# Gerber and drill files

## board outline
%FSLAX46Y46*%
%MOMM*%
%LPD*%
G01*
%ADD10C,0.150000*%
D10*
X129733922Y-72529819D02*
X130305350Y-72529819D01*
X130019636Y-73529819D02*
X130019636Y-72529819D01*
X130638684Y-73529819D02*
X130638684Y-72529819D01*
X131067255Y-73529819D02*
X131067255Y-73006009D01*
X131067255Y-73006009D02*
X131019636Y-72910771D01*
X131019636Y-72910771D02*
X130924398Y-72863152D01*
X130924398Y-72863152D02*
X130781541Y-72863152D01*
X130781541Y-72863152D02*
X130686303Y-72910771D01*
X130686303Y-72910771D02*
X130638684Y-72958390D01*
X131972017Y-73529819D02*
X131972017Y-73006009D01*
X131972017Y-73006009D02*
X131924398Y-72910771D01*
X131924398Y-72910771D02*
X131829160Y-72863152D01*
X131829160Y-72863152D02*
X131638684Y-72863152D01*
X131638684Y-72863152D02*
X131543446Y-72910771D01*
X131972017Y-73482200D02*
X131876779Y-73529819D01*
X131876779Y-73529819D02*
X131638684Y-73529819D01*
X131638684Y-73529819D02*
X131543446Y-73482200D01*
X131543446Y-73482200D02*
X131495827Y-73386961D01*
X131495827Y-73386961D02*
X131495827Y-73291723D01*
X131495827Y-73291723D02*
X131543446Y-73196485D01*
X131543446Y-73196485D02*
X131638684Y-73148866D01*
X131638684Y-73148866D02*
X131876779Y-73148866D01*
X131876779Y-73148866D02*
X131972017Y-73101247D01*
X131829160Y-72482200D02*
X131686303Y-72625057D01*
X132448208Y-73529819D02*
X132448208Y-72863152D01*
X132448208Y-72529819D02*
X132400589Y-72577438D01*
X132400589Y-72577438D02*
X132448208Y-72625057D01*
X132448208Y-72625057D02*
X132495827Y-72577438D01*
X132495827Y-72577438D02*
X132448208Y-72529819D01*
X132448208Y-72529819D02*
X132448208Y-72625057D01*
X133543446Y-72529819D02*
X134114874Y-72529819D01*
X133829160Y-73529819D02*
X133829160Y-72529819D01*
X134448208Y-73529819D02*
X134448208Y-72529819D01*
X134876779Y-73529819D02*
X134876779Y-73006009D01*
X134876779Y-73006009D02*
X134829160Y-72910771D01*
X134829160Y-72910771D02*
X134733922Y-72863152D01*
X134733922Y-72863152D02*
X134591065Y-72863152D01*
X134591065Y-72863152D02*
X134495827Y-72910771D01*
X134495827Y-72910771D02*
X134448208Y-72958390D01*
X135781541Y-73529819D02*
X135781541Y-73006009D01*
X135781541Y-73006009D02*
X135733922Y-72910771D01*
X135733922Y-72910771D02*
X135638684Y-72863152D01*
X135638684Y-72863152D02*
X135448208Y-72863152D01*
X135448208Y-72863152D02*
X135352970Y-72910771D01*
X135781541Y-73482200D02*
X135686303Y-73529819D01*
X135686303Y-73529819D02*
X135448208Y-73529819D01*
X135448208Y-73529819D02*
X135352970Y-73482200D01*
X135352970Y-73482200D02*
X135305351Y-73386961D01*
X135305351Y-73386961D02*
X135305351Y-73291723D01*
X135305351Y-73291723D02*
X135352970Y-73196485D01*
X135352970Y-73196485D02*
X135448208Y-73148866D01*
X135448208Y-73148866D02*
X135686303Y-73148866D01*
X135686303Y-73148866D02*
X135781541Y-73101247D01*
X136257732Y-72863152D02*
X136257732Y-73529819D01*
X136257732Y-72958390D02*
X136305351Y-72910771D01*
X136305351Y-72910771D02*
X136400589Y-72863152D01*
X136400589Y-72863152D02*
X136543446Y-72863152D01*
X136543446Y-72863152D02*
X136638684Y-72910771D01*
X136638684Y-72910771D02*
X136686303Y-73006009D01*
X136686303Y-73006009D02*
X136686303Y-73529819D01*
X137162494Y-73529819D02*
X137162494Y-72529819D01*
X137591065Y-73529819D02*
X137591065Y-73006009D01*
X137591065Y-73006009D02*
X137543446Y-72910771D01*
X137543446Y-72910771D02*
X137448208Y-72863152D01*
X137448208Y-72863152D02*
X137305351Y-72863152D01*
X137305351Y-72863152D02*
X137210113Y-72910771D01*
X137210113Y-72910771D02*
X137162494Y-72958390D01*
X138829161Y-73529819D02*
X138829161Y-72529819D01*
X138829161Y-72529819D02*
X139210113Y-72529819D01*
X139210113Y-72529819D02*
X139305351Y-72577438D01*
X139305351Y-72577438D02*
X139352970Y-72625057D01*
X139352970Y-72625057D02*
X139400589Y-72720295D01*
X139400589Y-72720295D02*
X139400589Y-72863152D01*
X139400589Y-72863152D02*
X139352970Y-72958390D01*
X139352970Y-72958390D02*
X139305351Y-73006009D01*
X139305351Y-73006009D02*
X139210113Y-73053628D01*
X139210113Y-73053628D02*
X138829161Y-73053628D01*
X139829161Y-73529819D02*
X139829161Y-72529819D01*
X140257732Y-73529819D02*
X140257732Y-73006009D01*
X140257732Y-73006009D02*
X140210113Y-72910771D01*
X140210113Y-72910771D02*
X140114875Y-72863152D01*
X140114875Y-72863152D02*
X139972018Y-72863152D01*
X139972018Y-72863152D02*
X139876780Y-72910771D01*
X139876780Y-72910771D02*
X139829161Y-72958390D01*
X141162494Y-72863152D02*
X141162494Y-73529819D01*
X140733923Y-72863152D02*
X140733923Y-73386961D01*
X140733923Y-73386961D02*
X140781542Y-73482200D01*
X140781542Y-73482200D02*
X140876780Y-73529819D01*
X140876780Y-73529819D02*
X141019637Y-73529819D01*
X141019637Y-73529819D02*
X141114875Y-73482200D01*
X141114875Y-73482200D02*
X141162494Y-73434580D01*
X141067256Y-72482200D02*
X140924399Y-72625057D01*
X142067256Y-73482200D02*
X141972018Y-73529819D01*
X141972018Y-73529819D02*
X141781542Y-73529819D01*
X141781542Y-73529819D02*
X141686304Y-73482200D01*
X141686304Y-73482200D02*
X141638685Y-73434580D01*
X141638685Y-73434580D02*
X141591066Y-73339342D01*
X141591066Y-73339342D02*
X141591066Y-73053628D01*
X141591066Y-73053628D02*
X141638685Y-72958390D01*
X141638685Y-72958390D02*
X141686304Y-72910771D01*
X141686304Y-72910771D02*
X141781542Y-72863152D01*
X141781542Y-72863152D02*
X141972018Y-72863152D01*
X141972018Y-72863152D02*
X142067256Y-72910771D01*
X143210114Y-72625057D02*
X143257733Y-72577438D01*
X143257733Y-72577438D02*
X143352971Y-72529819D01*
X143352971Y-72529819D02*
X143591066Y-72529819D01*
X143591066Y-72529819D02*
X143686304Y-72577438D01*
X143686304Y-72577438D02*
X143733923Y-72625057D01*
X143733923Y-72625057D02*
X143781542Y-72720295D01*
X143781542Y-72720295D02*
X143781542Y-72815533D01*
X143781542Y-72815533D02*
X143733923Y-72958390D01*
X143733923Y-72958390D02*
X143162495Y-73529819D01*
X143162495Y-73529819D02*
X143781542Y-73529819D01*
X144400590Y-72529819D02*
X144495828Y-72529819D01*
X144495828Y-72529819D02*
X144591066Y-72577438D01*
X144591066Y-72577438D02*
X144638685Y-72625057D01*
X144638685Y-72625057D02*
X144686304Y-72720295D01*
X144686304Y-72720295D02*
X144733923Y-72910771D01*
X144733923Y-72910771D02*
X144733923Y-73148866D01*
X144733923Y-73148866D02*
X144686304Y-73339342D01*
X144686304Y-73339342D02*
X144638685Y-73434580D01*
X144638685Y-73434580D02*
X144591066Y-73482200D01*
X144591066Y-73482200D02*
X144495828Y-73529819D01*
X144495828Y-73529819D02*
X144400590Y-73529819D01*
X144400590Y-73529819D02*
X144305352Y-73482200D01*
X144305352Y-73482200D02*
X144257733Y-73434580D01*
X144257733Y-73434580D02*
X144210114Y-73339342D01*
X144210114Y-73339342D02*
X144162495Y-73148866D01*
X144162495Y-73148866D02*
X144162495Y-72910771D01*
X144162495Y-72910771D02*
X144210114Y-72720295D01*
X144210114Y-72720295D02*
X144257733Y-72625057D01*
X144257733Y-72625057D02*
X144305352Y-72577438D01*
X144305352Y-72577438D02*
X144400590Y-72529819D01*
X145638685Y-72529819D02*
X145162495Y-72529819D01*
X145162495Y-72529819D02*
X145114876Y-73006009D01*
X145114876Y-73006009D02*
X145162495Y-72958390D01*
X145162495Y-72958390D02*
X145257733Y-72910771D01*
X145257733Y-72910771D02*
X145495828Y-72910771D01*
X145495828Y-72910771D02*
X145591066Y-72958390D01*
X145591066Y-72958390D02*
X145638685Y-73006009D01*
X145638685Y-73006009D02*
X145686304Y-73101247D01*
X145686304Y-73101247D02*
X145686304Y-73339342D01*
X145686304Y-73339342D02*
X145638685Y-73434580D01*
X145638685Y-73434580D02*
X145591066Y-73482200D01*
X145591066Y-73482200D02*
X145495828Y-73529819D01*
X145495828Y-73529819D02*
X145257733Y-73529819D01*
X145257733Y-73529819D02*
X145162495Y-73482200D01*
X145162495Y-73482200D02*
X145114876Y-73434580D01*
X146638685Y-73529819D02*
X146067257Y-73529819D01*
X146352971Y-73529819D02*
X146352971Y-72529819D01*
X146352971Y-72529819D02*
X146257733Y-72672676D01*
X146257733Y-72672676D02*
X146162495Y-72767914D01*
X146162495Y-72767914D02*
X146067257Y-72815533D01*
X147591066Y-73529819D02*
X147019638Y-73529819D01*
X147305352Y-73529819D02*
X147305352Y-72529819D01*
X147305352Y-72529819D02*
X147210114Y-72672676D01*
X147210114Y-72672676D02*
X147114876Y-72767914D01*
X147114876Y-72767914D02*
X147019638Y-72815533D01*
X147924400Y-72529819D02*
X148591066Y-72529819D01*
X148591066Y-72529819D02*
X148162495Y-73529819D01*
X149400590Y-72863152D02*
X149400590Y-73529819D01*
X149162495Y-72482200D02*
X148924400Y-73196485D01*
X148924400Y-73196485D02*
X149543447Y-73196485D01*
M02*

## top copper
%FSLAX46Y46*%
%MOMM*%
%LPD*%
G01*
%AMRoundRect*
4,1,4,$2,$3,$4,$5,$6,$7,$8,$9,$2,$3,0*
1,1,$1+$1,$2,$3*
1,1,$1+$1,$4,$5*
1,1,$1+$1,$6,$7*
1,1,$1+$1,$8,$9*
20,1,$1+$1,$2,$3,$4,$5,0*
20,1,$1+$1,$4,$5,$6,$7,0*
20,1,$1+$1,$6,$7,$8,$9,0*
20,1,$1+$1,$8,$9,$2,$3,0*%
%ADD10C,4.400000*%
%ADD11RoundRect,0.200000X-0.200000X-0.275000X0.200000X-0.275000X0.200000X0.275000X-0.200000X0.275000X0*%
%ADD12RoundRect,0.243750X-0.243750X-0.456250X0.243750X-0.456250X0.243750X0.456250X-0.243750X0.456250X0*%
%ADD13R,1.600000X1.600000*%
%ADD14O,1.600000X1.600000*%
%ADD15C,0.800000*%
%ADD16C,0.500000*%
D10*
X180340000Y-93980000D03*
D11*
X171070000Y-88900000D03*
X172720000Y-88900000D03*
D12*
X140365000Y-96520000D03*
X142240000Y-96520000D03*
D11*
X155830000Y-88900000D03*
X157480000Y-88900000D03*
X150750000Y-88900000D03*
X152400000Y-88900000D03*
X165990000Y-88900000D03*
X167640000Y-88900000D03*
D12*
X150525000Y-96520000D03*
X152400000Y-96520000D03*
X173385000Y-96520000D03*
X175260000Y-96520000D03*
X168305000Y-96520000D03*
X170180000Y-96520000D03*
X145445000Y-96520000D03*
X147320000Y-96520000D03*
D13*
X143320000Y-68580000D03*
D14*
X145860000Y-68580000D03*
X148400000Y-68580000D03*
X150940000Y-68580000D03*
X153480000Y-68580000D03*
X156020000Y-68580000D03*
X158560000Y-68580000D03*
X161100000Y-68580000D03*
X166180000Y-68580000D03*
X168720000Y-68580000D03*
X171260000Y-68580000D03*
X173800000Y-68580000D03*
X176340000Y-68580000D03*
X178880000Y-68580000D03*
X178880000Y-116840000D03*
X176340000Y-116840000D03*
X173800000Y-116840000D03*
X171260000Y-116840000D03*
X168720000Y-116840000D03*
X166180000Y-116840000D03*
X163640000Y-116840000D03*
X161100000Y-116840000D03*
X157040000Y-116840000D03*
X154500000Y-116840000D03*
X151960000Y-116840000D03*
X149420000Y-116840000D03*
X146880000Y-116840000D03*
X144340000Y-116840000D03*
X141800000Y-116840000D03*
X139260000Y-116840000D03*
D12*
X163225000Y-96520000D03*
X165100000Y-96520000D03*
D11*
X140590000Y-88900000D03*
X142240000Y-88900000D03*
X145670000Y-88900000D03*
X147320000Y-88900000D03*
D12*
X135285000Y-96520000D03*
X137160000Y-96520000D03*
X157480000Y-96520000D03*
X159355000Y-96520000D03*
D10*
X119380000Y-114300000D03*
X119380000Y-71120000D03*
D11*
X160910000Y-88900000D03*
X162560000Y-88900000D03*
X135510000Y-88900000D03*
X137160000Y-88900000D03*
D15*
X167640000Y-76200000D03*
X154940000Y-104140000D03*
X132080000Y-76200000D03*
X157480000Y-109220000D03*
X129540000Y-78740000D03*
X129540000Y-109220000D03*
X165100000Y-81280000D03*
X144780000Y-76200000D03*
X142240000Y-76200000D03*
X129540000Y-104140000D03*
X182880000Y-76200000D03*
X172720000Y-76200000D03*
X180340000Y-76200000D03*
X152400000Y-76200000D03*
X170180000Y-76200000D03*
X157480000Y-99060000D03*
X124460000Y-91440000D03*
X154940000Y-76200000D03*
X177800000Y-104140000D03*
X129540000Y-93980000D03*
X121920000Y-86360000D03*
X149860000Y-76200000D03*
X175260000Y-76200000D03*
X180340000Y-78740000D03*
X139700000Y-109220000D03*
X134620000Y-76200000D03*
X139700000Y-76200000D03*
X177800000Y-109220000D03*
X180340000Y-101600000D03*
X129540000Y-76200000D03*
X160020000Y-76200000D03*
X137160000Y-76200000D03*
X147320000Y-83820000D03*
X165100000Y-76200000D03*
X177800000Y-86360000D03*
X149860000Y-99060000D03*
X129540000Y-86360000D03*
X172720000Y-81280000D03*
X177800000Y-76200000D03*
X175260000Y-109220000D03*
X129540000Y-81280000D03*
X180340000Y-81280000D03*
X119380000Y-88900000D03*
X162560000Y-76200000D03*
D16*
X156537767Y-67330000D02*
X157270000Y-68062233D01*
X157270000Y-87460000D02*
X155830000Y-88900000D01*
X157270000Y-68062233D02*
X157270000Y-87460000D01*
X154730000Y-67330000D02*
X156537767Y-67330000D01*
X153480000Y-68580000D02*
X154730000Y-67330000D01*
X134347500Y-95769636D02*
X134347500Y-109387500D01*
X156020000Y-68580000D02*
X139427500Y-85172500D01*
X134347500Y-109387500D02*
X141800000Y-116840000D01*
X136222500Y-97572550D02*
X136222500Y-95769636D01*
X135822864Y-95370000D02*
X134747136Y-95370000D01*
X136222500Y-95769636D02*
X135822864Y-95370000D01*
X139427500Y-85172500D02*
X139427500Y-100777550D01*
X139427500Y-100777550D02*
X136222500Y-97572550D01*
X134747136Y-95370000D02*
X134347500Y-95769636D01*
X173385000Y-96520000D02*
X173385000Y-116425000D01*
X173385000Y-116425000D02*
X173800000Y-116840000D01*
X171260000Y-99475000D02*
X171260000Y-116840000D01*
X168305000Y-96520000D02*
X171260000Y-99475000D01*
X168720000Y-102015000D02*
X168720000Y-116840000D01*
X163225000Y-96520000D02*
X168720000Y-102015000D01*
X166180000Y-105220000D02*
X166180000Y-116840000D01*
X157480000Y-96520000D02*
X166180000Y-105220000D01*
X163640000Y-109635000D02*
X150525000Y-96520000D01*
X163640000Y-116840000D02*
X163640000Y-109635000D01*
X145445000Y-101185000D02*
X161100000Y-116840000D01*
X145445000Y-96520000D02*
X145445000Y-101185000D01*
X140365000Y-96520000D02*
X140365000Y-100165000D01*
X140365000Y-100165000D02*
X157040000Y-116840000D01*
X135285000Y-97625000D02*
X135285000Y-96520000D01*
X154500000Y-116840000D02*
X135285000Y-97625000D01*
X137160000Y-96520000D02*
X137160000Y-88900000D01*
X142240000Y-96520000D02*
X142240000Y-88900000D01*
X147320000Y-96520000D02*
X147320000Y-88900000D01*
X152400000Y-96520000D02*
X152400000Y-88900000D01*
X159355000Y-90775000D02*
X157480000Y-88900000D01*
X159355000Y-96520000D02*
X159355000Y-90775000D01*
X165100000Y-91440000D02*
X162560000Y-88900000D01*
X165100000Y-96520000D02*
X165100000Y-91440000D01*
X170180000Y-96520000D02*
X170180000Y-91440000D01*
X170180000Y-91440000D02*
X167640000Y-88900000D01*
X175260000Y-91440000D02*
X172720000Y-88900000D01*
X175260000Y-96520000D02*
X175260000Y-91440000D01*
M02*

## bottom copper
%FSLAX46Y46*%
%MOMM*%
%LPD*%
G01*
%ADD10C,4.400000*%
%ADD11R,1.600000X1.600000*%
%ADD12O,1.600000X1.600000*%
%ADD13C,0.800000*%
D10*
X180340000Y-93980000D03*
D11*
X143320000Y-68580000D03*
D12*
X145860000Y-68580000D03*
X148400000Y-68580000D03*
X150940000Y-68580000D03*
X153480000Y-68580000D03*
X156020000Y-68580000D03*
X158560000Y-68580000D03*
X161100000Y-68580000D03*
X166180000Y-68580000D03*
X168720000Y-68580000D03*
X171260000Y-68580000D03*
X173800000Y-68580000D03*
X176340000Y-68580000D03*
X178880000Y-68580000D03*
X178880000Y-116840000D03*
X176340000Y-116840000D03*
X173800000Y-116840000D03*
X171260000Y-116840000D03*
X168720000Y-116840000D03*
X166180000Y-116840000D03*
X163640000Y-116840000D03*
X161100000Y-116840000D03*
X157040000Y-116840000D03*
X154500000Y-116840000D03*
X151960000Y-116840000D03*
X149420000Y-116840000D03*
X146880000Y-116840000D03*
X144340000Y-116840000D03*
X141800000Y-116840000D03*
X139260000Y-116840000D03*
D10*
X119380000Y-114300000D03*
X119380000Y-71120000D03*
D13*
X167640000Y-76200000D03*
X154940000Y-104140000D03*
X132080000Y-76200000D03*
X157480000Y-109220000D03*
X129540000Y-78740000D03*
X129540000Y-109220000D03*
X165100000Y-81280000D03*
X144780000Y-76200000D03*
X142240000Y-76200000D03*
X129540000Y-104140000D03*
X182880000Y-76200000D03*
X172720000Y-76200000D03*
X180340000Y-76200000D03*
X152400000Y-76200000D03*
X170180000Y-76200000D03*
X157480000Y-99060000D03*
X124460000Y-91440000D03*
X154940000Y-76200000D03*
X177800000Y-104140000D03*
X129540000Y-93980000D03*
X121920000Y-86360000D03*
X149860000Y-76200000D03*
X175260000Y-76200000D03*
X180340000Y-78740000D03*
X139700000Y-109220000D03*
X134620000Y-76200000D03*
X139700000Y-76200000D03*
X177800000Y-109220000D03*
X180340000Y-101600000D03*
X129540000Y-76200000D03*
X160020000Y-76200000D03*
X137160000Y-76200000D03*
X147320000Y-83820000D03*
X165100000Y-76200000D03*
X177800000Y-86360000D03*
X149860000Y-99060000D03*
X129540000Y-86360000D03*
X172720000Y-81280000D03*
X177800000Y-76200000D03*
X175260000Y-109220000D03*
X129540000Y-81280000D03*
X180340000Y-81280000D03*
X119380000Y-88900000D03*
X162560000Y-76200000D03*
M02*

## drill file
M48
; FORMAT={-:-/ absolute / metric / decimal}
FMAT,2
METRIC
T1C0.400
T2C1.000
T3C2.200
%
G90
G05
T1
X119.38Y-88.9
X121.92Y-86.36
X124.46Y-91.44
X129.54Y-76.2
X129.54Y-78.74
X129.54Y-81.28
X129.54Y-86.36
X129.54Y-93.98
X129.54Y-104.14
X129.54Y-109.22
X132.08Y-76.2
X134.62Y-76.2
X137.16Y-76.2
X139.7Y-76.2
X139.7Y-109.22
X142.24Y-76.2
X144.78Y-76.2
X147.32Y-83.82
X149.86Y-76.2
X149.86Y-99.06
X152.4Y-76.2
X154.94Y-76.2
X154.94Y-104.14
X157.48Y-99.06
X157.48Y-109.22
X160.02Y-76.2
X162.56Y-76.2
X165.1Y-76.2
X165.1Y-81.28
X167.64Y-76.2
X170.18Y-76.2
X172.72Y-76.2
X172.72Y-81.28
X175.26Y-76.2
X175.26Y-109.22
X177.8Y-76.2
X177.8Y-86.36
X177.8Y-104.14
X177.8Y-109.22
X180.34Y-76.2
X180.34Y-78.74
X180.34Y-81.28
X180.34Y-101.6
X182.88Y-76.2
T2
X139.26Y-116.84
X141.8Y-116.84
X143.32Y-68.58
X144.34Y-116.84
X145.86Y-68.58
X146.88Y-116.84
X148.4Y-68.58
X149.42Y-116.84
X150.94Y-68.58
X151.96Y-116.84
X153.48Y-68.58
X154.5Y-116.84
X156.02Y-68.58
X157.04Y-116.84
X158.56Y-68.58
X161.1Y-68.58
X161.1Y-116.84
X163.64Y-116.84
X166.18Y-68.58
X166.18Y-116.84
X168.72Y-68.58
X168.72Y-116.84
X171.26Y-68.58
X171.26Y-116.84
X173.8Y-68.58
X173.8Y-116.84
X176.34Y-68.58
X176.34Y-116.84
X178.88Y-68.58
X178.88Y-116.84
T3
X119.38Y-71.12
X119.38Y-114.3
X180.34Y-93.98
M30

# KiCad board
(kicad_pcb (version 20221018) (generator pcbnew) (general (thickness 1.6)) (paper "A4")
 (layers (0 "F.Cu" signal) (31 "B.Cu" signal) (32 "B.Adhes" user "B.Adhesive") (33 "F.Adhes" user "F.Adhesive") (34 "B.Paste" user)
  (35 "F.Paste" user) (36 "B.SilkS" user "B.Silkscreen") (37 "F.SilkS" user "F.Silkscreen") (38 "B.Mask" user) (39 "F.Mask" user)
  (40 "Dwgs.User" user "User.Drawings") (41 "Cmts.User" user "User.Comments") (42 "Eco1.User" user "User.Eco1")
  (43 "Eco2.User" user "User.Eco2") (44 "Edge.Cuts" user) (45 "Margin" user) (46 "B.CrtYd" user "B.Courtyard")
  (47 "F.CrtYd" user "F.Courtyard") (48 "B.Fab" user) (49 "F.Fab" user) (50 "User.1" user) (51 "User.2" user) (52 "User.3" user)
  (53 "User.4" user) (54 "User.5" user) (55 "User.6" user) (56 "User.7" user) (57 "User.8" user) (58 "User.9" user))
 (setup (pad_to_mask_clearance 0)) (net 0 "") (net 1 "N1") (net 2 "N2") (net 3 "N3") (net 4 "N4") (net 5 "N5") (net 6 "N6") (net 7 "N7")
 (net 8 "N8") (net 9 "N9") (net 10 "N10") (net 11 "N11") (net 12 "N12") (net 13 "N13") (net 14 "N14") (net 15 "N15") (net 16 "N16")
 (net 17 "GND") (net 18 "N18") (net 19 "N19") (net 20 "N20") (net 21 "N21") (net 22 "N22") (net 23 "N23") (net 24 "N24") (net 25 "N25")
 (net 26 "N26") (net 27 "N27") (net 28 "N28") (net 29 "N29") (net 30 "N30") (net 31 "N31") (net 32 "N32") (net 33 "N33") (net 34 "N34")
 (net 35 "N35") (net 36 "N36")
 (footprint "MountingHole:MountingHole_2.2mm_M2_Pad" (layer "F.Cu") (at 180.34 93.98)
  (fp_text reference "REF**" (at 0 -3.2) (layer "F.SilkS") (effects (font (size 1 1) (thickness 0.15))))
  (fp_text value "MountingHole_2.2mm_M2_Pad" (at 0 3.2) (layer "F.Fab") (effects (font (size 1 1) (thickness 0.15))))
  (pad "1" thru_hole circle (at 0 0) (size 4.4 4.4) (drill 2.2) (layers "*.Cu" "*.Mask")))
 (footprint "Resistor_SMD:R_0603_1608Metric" (layer "F.Cu") (at 171.895 88.9)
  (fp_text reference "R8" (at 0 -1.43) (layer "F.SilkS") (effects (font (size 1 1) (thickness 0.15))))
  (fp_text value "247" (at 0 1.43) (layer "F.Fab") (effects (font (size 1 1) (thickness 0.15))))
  (pad "1" smd roundrect (at -0.825 0) (size 0.8 0.95) (layers "F.Cu" "F.Paste" "F.Mask") (roundrect_rratio 0.25) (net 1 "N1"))
  (pad "2" smd roundrect (at 0.825 0) (size 0.8 0.95) (layers "F.Cu" "F.Paste" "F.Mask") (roundrect_rratio 0.25) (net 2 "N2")))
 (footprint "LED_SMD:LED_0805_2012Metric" (layer "F.Cu") (at 141.3025 96.52)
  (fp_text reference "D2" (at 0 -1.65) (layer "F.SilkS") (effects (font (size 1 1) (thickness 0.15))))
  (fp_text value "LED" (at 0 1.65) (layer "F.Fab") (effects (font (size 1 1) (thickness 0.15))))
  (pad "1" smd roundrect (at -0.9375 0) (size 0.975 1.4) (layers "F.Cu" "F.Paste" "F.Mask") (roundrect_rratio 0.25) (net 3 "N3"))
  (pad "2" smd roundrect (at 0.9375 0) (size 0.975 1.4) (layers "F.Cu" "F.Paste" "F.Mask") (roundrect_rratio 0.25) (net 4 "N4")))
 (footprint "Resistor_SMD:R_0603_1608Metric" (layer "F.Cu") (at 156.655 88.9)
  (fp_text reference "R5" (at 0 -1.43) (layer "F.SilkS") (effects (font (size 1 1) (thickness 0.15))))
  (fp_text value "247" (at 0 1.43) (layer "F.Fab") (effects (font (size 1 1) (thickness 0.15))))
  (pad "1" smd roundrect (at -0.825 0) (size 0.8 0.95) (layers "F.Cu" "F.Paste" "F.Mask") (roundrect_rratio 0.25) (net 1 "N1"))
  (pad "2" smd roundrect (at 0.825 0) (size 0.8 0.95) (layers "F.Cu" "F.Paste" "F.Mask") (roundrect_rratio 0.25) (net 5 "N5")))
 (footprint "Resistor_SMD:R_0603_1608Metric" (layer "F.Cu") (at 151.575 88.9)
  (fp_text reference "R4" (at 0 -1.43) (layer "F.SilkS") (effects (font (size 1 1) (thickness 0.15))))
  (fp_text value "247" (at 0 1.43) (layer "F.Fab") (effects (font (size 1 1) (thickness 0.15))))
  (pad "1" smd roundrect (at -0.825 0) (size 0.8 0.95) (layers "F.Cu" "F.Paste" "F.Mask") (roundrect_rratio 0.25) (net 1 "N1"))
  (pad "2" smd roundrect (at 0.825 0) (size 0.8 0.95) (layers "F.Cu" "F.Paste" "F.Mask") (roundrect_rratio 0.25) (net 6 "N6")))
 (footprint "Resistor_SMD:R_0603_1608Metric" (layer "F.Cu") (at 166.815 88.9)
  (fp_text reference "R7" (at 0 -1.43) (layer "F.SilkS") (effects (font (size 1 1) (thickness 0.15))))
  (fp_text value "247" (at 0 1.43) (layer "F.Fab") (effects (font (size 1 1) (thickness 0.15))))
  (pad "1" smd roundrect (at -0.825 0) (size 0.8 0.95) (layers "F.Cu" "F.Paste" "F.Mask") (roundrect_rratio 0.25) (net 1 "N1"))
  (pad "2" smd roundrect (at 0.825 0) (size 0.8 0.95) (layers "F.Cu" "F.Paste" "F.Mask") (roundrect_rratio 0.25) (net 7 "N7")))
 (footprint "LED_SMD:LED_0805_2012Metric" (layer "F.Cu") (at 151.4625 96.52)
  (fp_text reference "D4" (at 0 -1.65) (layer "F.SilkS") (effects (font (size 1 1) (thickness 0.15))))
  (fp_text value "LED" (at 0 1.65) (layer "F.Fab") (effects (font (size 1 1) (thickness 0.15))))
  (pad "1" smd roundrect (at -0.9375 0) (size 0.975 1.4) (layers "F.Cu" "F.Paste" "F.Mask") (roundrect_rratio 0.25) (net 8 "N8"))
  (pad "2" smd roundrect (at 0.9375 0) (size 0.975 1.4) (layers "F.Cu" "F.Paste" "F.Mask") (roundrect_rratio 0.25) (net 6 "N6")))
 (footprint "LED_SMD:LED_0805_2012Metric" (layer "F.Cu") (at 174.3225 96.52)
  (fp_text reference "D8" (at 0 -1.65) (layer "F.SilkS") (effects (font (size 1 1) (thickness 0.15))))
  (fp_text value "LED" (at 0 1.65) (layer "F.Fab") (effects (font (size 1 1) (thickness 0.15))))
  (pad "1" smd roundrect (at -0.9375 0) (size 0.975 1.4) (layers "F.Cu" "F.Paste" "F.Mask") (roundrect_rratio 0.25) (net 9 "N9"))
  (pad "2" smd roundrect (at 0.9375 0) (size 0.975 1.4) (layers "F.Cu" "F.Paste" "F.Mask") (roundrect_rratio 0.25) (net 2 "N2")))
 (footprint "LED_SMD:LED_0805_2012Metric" (layer "F.Cu") (at 169.2425 96.52)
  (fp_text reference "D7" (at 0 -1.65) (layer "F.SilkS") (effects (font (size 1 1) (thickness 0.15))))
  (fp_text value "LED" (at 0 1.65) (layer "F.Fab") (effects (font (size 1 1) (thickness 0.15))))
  (pad "1" smd roundrect (at -0.9375 0) (size 0.975 1.4) (layers "F.Cu" "F.Paste" "F.Mask") (roundrect_rratio 0.25) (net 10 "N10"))
  (pad "2" smd roundrect (at 0.9375 0) (size 0.975 1.4) (layers "F.Cu" "F.Paste" "F.Mask") (roundrect_rratio 0.25) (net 7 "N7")))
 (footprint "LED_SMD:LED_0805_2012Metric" (layer "F.Cu") (at 146.3825 96.52)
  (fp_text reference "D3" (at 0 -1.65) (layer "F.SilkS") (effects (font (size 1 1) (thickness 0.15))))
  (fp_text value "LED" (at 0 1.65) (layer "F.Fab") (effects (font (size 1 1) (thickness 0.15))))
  (pad "1" smd roundrect (at -0.9375 0) (size 0.975 1.4) (layers "F.Cu" "F.Paste" "F.Mask") (roundrect_rratio 0.25) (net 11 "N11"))
  (pad "2" smd roundrect (at 0.9375 0) (size 0.975 1.4) (layers "F.Cu" "F.Paste" "F.Mask") (roundrect_rratio 0.25) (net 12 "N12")))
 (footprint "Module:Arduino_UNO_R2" (layer "F.Cu") (at 143.32 68.58)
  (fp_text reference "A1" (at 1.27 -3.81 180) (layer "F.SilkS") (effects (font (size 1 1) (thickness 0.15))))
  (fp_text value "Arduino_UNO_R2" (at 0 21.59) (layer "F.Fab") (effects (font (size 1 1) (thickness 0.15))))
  (pad "1" thru_hole rect (at 0 0 90) (size 1.6 1.6) (drill 1) (layers "*.Cu" "*.Mask") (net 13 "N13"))
  (pad "2" thru_hole oval (at 2.54 0 90) (size 1.6 1.6) (drill 1) (layers "*.Cu" "*.Mask") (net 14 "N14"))
  (pad "3" thru_hole oval (at 5.08 0 90) (size 1.6 1.6) (drill 1) (layers "*.Cu" "*.Mask") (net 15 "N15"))
  (pad "4" thru_hole oval (at 7.62 0 90) (size 1.6 1.6) (drill 1) (layers "*.Cu" "*.Mask") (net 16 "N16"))
  (pad "5" thru_hole oval (at 10.16 0 90) (size 1.6 1.6) (drill 1) (layers "*.Cu" "*.Mask") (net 1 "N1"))
  (pad "6" thru_hole oval (at 12.7 0 90) (size 1.6 1.6) (drill 1) (layers "*.Cu" "*.Mask") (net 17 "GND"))
  (pad "7" thru_hole oval (at 15.24 0 90) (size 1.6 1.6) (drill 1) (layers "*.Cu" "*.Mask") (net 17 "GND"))
  (pad "8" thru_hole oval (at 17.78 0 90) (size 1.6 1.6) (drill 1) (layers "*.Cu" "*.Mask") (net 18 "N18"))
  (pad "9" thru_hole oval (at 22.86 0 90) (size 1.6 1.6) (drill 1) (layers "*.Cu" "*.Mask") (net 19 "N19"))
  (pad "10" thru_hole oval (at 25.4 0 90) (size 1.6 1.6) (drill 1) (layers "*.Cu" "*.Mask") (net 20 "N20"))
  (pad "11" thru_hole oval (at 27.94 0 90) (size 1.6 1.6) (drill 1) (layers "*.Cu" "*.Mask") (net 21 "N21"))
  (pad "12" thru_hole oval (at 30.48 0 90) (size 1.6 1.6) (drill 1) (layers "*.Cu" "*.Mask") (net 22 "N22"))
  (pad "13" thru_hole oval (at 33.02 0 90) (size 1.6 1.6) (drill 1) (layers "*.Cu" "*.Mask") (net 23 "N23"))
  (pad "14" thru_hole oval (at 35.56 0 90) (size 1.6 1.6) (drill 1) (layers "*.Cu" "*.Mask") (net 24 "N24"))
  (pad "15" thru_hole oval (at 35.56 48.26 90) (size 1.6 1.6) (drill 1) (layers "*.Cu" "*.Mask") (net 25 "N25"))
  (pad "16" thru_hole oval (at 33.02 48.26 90) (size 1.6 1.6) (drill 1) (layers "*.Cu" "*.Mask") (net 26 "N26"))
  (pad "17" thru_hole oval (at 30.48 48.26 90) (size 1.6 1.6) (drill 1) (layers "*.Cu" "*.Mask") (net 9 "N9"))
  (pad "18" thru_hole oval (at 27.94 48.26 90) (size 1.6 1.6) (drill 1) (layers "*.Cu" "*.Mask") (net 10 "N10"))
  (pad "19" thru_hole oval (at 25.4 48.26 90) (size 1.6 1.6) (drill 1) (layers "*.Cu" "*.Mask") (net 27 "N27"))
  (pad "20" thru_hole oval (at 22.86 48.26 90) (size 1.6 1.6) (drill 1) (layers "*.Cu" "*.Mask") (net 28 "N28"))
  (pad "21" thru_hole oval (at 20.32 48.26 90) (size 1.6 1.6) (drill 1) (layers "*.Cu" "*.Mask") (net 8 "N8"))
  (pad "22" thru_hole oval (at 17.78 48.26 90) (size 1.6 1.6) (drill 1) (layers "*.Cu" "*.Mask") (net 11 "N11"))
  (pad "23" thru_hole oval (at 13.72 48.26 90) (size 1.6 1.6) (drill 1) (layers "*.Cu" "*.Mask") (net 3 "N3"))
  (pad "24" thru_hole oval (at 11.18 48.26 90) (size 1.6 1.6) (drill 1) (layers "*.Cu" "*.Mask") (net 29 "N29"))
  (pad "25" thru_hole oval (at 8.64 48.26 90) (size 1.6 1.6) (drill 1) (layers "*.Cu" "*.Mask") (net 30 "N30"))
  (pad "26" thru_hole oval (at 6.1 48.26 90) (size 1.6 1.6) (drill 1) (layers "*.Cu" "*.Mask") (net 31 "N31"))
  (pad "27" thru_hole oval (at 3.56 48.26 90) (size 1.6 1.6) (drill 1) (layers "*.Cu" "*.Mask") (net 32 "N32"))
  (pad "28" thru_hole oval (at 1.02 48.26 90) (size 1.6 1.6) (drill 1) (layers "*.Cu" "*.Mask") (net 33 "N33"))
  (pad "29" thru_hole oval (at -1.52 48.26 90) (size 1.6 1.6) (drill 1) (layers "*.Cu" "*.Mask") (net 17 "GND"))
  (pad "30" thru_hole oval (at -4.06 48.26 90) (size 1.6 1.6) (drill 1) (layers "*.Cu" "*.Mask") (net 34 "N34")))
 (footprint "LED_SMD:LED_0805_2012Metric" (layer "F.Cu") (at 164.1625 96.52)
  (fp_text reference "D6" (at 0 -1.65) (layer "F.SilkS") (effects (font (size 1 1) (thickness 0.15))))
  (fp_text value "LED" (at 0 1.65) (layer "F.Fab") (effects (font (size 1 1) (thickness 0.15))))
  (pad "1" smd roundrect (at -0.9375 0) (size 0.975 1.4) (layers "F.Cu" "F.Paste" "F.Mask") (roundrect_rratio 0.25) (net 27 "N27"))
  (pad "2" smd roundrect (at 0.9375 0) (size 0.975 1.4) (layers "F.Cu" "F.Paste" "F.Mask") (roundrect_rratio 0.25) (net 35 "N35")))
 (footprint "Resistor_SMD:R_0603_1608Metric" (layer "F.Cu") (at 141.415 88.9)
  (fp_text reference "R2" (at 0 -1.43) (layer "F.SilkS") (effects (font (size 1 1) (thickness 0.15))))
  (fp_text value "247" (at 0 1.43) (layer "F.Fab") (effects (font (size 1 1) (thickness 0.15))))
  (pad "1" smd roundrect (at -0.825 0) (size 0.8 0.95) (layers "F.Cu" "F.Paste" "F.Mask") (roundrect_rratio 0.25) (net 1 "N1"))
  (pad "2" smd roundrect (at 0.825 0) (size 0.8 0.95) (layers "F.Cu" "F.Paste" "F.Mask") (roundrect_rratio 0.25) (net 4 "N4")))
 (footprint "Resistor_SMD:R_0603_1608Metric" (layer "F.Cu") (at 146.495 88.9)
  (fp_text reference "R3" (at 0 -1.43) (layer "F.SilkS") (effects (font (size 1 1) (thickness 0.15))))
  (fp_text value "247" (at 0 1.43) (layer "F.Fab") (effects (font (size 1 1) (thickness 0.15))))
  (pad "1" smd roundrect (at -0.825 0) (size 0.8 0.95) (layers "F.Cu" "F.Paste" "F.Mask") (roundrect_rratio 0.25) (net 1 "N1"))
  (pad "2" smd roundrect (at 0.825 0) (size 0.8 0.95) (layers "F.Cu" "F.Paste" "F.Mask") (roundrect_rratio 0.25) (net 12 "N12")))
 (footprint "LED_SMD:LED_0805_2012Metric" (layer "F.Cu") (at 136.2225 96.52)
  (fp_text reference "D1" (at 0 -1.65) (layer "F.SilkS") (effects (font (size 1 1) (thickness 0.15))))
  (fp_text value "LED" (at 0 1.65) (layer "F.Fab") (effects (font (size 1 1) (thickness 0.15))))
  (pad "1" smd roundrect (at -0.9375 0) (size 0.975 1.4) (layers "F.Cu" "F.Paste" "F.Mask") (roundrect_rratio 0.25) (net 29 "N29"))
  (pad "2" smd roundrect (at 0.9375 0) (size 0.975 1.4) (layers "F.Cu" "F.Paste" "F.Mask") (roundrect_rratio 0.25) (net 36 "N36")))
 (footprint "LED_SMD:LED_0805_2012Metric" (layer "F.Cu") (at 158.4175 96.52)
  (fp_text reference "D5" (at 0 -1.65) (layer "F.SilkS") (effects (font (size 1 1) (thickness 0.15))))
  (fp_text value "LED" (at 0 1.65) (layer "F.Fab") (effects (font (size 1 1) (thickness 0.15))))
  (pad "1" smd roundrect (at -0.9375 0) (size 0.975 1.4) (layers "F.Cu" "F.Paste" "F.Mask") (roundrect_rratio 0.25) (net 28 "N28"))
  (pad "2" smd roundrect (at 0.9375 0) (size 0.975 1.4) (layers "F.Cu" "F.Paste" "F.Mask") (roundrect_rratio 0.25) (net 5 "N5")))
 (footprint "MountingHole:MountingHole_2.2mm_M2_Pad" (layer "F.Cu") (at 119.38 114.3)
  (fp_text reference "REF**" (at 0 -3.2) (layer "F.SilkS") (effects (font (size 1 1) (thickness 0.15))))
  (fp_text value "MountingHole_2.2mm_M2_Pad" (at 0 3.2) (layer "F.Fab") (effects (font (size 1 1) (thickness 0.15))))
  (pad "1" thru_hole circle (at 0 0) (size 4.4 4.4) (drill 2.2) (layers "*.Cu" "*.Mask")))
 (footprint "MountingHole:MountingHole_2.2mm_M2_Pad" (layer "F.Cu") (at 119.38 71.12)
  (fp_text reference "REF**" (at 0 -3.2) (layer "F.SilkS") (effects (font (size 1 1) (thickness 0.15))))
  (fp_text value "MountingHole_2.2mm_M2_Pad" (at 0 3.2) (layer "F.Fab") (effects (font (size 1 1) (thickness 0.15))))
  (pad "1" thru_hole circle (at 0 0) (size 4.4 4.4) (drill 2.2) (layers "*.Cu" "*.Mask")))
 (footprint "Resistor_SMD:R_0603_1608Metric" (layer "F.Cu") (at 161.735 88.9)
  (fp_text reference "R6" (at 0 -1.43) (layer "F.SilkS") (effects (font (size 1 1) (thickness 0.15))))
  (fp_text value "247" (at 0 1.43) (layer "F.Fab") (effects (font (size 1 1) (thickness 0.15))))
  (pad "1" smd roundrect (at -0.825 0) (size 0.8 0.95) (layers "F.Cu" "F.Paste" "F.Mask") (roundrect_rratio 0.25) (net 1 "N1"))
  (pad "2" smd roundrect (at 0.825 0) (size 0.8 0.95) (layers "F.Cu" "F.Paste" "F.Mask") (roundrect_rratio 0.25) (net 35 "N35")))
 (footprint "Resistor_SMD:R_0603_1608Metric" (layer "F.Cu") (at 136.335 88.9)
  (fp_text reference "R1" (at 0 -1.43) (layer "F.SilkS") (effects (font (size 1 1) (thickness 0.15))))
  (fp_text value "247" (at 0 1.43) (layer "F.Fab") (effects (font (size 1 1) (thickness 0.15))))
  (pad "1" smd roundrect (at -0.825 0) (size 0.8 0.95) (layers "F.Cu" "F.Paste" "F.Mask") (roundrect_rratio 0.25) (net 1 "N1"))
  (pad "2" smd roundrect (at 0.825 0) (size 0.8 0.95) (layers "F.Cu" "F.Paste" "F.Mask") (roundrect_rratio 0.25) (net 36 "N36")))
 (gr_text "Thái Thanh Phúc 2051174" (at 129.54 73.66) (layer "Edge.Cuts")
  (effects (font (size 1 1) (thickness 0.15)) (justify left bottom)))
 (via (at 167.64 76.2) (size 0.8) (drill 0.4) (layers "F.Cu" "B.Cu") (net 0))
 (via (at 154.94 104.14) (size 0.8) (drill 0.4) (layers "F.Cu" "B.Cu") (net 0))
 (via (at 132.08 76.2) (size 0.8) (drill 0.4) (layers "F.Cu" "B.Cu") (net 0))
 (via (at 157.48 109.22) (size 0.8) (drill 0.4) (layers "F.Cu" "B.Cu") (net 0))
 (via (at 129.54 78.74) (size 0.8) (drill 0.4) (layers "F.Cu" "B.Cu") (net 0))
 (via (at 129.54 109.22) (size 0.8) (drill 0.4) (layers "F.Cu" "B.Cu") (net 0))
 (via (at 165.1 81.28) (size 0.8) (drill 0.4) (layers "F.Cu" "B.Cu") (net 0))
 (via (at 144.78 76.2) (size 0.8) (drill 0.4) (layers "F.Cu" "B.Cu") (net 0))
 (via (at 142.24 76.2) (size 0.8) (drill 0.4) (layers "F.Cu" "B.Cu") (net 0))
 (via (at 129.54 104.14) (size 0.8) (drill 0.4) (layers "F.Cu" "B.Cu") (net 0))
 (via (at 182.88 76.2) (size 0.8) (drill 0.4) (layers "F.Cu" "B.Cu") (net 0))
 (via (at 172.72 76.2) (size 0.8) (drill 0.4) (layers "F.Cu" "B.Cu") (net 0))
 (via (at 180.34 76.2) (size 0.8) (drill 0.4) (layers "F.Cu" "B.Cu") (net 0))
 (via (at 152.4 76.2) (size 0.8) (drill 0.4) (layers "F.Cu" "B.Cu") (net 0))
 (via (at 170.18 76.2) (size 0.8) (drill 0.4) (layers "F.Cu" "B.Cu") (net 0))
 (via (at 157.48 99.06) (size 0.8) (drill 0.4) (layers "F.Cu" "B.Cu") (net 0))
 (via (at 124.46 91.44) (size 0.8) (drill 0.4) (layers "F.Cu" "B.Cu") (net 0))
 (via (at 154.94 76.2) (size 0.8) (drill 0.4) (layers "F.Cu" "B.Cu") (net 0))
 (via (at 177.8 104.14) (size 0.8) (drill 0.4) (layers "F.Cu" "B.Cu") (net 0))
 (via (at 129.54 93.98) (size 0.8) (drill 0.4) (layers "F.Cu" "B.Cu") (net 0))
 (via (at 121.92 86.36) (size 0.8) (drill 0.4) (layers "F.Cu" "B.Cu") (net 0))
 (via (at 149.86 76.2) (size 0.8) (drill 0.4) (layers "F.Cu" "B.Cu") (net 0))
 (via (at 175.26 76.2) (size 0.8) (drill 0.4) (layers "F.Cu" "B.Cu") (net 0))
 (via (at 180.34 78.74) (size 0.8) (drill 0.4) (layers "F.Cu" "B.Cu") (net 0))
 (via (at 139.7 109.22) (size 0.8) (drill 0.4) (layers "F.Cu" "B.Cu") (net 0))
 (via (at 134.62 76.2) (size 0.8) (drill 0.4) (layers "F.Cu" "B.Cu") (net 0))
 (via (at 139.7 76.2) (size 0.8) (drill 0.4) (layers "F.Cu" "B.Cu") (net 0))
 (via (at 177.8 109.22) (size 0.8) (drill 0.4) (layers "F.Cu" "B.Cu") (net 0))
 (via (at 180.34 101.6) (size 0.8) (drill 0.4) (layers "F.Cu" "B.Cu") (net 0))
 (via (at 129.54 76.2) (size 0.8) (drill 0.4) (layers "F.Cu" "B.Cu") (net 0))
 (via (at 160.02 76.2) (size 0.8) (drill 0.4) (layers "F.Cu" "B.Cu") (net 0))
 (via (at 137.16 76.2) (size 0.8) (drill 0.4) (layers "F.Cu" "B.Cu") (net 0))
 (via (at 147.32 83.82) (size 0.8) (drill 0.4) (layers "F.Cu" "B.Cu") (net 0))
 (via (at 165.1 76.2) (size 0.8) (drill 0.4) (layers "F.Cu" "B.Cu") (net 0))
 (via (at 177.8 86.36) (size 0.8) (drill 0.4) (layers "F.Cu" "B.Cu") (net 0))
 (via (at 149.86 99.06) (size 0.8) (drill 0.4) (layers "F.Cu" "B.Cu") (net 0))
 (via (at 129.54 86.36) (size 0.8) (drill 0.4) (layers "F.Cu" "B.Cu") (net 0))
 (via (at 172.72 81.28) (size 0.8) (drill 0.4) (layers "F.Cu" "B.Cu") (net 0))
 (via (at 177.8 76.2) (size 0.8) (drill 0.4) (layers "F.Cu" "B.Cu") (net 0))
 (via (at 175.26 109.22) (size 0.8) (drill 0.4) (layers "F.Cu" "B.Cu") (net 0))
 (via (at 129.54 81.28) (size 0.8) (drill 0.4) (layers "F.Cu" "B.Cu") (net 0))
 (via (at 180.34 81.28) (size 0.8) (drill 0.4) (layers "F.Cu" "B.Cu") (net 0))
 (via (at 119.38 88.9) (size 0.8) (drill 0.4) (layers "F.Cu" "B.Cu") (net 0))
 (via (at 162.56 76.2) (size 0.8) (drill 0.4) (layers "F.Cu" "B.Cu") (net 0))
 (segment (start 156.537767 67.33) (end 157.27 68.062233) (width 0.5) (layer "F.Cu") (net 1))
 (segment (start 157.27 87.46) (end 155.83 88.9) (width 0.5) (layer "F.Cu") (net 1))
 (segment (start 157.27 68.062233) (end 157.27 87.46) (width 0.5) (layer "F.Cu") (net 1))
 (segment (start 154.73 67.33) (end 156.537767 67.33) (width 0.5) (layer "F.Cu") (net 1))
 (segment (start 153.48 68.58) (end 154.73 67.33) (width 0.5) (layer "F.Cu") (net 1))
 (segment (start 134.3475 95.769636) (end 134.3475 109.3875) (width 0.5) (layer "F.Cu") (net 17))
 (segment (start 156.02 68.58) (end 139.4275 85.1725) (width 0.5) (layer "F.Cu") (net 17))
 (segment (start 134.3475 109.3875) (end 141.8 116.84) (width 0.5) (layer "F.Cu") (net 17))
 (segment (start 136.2225 97.57255) (end 136.2225 95.769636) (width 0.5) (layer "F.Cu") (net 17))
 (segment (start 135.822864 95.37) (end 134.747136 95.37) (width 0.5) (layer "F.Cu") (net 17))
 (segment (start 136.2225 95.769636) (end 135.822864 95.37) (width 0.5) (layer "F.Cu") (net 17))
 (segment (start 139.4275 85.1725) (end 139.4275 100.77755) (width 0.5) (layer "F.Cu") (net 17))
 (segment (start 139.4275 100.77755) (end 136.2225 97.57255) (width 0.5) (layer "F.Cu") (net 17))
 (segment (start 134.747136 95.37) (end 134.3475 95.769636) (width 0.5) (layer "F.Cu") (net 17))
 (segment (start 173.385 96.52) (end 173.385 116.425) (width 0.5) (layer "F.Cu") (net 9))
 (segment (start 173.385 116.425) (end 173.8 116.84) (width 0.5) (layer "F.Cu") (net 9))
 (segment (start 171.26 99.475) (end 171.26 116.84) (width 0.5) (layer "F.Cu") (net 10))
 (segment (start 168.305 96.52) (end 171.26 99.475) (width 0.5) (layer "F.Cu") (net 10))
 (segment (start 168.72 102.015) (end 168.72 116.84) (width 0.5) (layer "F.Cu") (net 27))
 (segment (start 163.225 96.52) (end 168.72 102.015) (width 0.5) (layer "F.Cu") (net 27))
 (segment (start 166.18 105.22) (end 166.18 116.84) (width 0.5) (layer "F.Cu") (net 28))
 (segment (start 157.48 96.52) (end 166.18 105.22) (width 0.5) (layer "F.Cu") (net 28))
 (segment (start 163.64 109.635) (end 150.525 96.52) (width 0.5) (layer "F.Cu") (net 8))
 (segment (start 163.64 116.84) (end 163.64 109.635) (width 0.5) (layer "F.Cu") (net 8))
 (segment (start 145.445 101.185) (end 161.1 116.84) (width 0.5) (layer "F.Cu") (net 11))
 (segment (start 145.445 96.52) (end 145.445 101.185) (width 0.5) (layer "F.Cu") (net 11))
 (segment (start 140.365 96.52) (end 140.365 100.165) (width 0.5) (layer "F.Cu") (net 3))
 (segment (start 140.365 100.165) (end 157.04 116.84) (width 0.5) (layer "F.Cu") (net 3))
 (segment (start 135.285 97.625) (end 135.285 96.52) (width 0.5) (layer "F.Cu") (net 29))
 (segment (start 154.5 116.84) (end 135.285 97.625) (width 0.5) (layer "F.Cu") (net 29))
 (segment (start 137.16 96.52) (end 137.16 88.9) (width 0.5) (layer "F.Cu") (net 36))
 (segment (start 142.24 96.52) (end 142.24 88.9) (width 0.5) (layer "F.Cu") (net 4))
 (segment (start 147.32 96.52) (end 147.32 88.9) (width 0.5) (layer "F.Cu") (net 12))
 (segment (start 152.4 96.52) (end 152.4 88.9) (width 0.5) (layer "F.Cu") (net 6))
 (segment (start 159.355 90.775) (end 157.48 88.9) (width 0.5) (layer "F.Cu") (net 5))
 (segment (start 159.355 96.52) (end 159.355 90.775) (width 0.5) (layer "F.Cu") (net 5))
 (segment (start 165.1 91.44) (end 162.56 88.9) (width 0.5) (layer "F.Cu") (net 35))
 (segment (start 165.1 96.52) (end 165.1 91.44) (width 0.5) (layer "F.Cu") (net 35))
 (segment (start 170.18 96.52) (end 170.18 91.44) (width 0.5) (layer "F.Cu") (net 7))
 (segment (start 170.18 91.44) (end 167.64 88.9) (width 0.5) (layer "F.Cu") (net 7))
 (segment (start 175.26 91.44) (end 172.72 88.9) (width 0.5) (layer "F.Cu") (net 2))
 (segment (start 175.26 96.52) (end 175.26 91.44) (width 0.5) (layer "F.Cu") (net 2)))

